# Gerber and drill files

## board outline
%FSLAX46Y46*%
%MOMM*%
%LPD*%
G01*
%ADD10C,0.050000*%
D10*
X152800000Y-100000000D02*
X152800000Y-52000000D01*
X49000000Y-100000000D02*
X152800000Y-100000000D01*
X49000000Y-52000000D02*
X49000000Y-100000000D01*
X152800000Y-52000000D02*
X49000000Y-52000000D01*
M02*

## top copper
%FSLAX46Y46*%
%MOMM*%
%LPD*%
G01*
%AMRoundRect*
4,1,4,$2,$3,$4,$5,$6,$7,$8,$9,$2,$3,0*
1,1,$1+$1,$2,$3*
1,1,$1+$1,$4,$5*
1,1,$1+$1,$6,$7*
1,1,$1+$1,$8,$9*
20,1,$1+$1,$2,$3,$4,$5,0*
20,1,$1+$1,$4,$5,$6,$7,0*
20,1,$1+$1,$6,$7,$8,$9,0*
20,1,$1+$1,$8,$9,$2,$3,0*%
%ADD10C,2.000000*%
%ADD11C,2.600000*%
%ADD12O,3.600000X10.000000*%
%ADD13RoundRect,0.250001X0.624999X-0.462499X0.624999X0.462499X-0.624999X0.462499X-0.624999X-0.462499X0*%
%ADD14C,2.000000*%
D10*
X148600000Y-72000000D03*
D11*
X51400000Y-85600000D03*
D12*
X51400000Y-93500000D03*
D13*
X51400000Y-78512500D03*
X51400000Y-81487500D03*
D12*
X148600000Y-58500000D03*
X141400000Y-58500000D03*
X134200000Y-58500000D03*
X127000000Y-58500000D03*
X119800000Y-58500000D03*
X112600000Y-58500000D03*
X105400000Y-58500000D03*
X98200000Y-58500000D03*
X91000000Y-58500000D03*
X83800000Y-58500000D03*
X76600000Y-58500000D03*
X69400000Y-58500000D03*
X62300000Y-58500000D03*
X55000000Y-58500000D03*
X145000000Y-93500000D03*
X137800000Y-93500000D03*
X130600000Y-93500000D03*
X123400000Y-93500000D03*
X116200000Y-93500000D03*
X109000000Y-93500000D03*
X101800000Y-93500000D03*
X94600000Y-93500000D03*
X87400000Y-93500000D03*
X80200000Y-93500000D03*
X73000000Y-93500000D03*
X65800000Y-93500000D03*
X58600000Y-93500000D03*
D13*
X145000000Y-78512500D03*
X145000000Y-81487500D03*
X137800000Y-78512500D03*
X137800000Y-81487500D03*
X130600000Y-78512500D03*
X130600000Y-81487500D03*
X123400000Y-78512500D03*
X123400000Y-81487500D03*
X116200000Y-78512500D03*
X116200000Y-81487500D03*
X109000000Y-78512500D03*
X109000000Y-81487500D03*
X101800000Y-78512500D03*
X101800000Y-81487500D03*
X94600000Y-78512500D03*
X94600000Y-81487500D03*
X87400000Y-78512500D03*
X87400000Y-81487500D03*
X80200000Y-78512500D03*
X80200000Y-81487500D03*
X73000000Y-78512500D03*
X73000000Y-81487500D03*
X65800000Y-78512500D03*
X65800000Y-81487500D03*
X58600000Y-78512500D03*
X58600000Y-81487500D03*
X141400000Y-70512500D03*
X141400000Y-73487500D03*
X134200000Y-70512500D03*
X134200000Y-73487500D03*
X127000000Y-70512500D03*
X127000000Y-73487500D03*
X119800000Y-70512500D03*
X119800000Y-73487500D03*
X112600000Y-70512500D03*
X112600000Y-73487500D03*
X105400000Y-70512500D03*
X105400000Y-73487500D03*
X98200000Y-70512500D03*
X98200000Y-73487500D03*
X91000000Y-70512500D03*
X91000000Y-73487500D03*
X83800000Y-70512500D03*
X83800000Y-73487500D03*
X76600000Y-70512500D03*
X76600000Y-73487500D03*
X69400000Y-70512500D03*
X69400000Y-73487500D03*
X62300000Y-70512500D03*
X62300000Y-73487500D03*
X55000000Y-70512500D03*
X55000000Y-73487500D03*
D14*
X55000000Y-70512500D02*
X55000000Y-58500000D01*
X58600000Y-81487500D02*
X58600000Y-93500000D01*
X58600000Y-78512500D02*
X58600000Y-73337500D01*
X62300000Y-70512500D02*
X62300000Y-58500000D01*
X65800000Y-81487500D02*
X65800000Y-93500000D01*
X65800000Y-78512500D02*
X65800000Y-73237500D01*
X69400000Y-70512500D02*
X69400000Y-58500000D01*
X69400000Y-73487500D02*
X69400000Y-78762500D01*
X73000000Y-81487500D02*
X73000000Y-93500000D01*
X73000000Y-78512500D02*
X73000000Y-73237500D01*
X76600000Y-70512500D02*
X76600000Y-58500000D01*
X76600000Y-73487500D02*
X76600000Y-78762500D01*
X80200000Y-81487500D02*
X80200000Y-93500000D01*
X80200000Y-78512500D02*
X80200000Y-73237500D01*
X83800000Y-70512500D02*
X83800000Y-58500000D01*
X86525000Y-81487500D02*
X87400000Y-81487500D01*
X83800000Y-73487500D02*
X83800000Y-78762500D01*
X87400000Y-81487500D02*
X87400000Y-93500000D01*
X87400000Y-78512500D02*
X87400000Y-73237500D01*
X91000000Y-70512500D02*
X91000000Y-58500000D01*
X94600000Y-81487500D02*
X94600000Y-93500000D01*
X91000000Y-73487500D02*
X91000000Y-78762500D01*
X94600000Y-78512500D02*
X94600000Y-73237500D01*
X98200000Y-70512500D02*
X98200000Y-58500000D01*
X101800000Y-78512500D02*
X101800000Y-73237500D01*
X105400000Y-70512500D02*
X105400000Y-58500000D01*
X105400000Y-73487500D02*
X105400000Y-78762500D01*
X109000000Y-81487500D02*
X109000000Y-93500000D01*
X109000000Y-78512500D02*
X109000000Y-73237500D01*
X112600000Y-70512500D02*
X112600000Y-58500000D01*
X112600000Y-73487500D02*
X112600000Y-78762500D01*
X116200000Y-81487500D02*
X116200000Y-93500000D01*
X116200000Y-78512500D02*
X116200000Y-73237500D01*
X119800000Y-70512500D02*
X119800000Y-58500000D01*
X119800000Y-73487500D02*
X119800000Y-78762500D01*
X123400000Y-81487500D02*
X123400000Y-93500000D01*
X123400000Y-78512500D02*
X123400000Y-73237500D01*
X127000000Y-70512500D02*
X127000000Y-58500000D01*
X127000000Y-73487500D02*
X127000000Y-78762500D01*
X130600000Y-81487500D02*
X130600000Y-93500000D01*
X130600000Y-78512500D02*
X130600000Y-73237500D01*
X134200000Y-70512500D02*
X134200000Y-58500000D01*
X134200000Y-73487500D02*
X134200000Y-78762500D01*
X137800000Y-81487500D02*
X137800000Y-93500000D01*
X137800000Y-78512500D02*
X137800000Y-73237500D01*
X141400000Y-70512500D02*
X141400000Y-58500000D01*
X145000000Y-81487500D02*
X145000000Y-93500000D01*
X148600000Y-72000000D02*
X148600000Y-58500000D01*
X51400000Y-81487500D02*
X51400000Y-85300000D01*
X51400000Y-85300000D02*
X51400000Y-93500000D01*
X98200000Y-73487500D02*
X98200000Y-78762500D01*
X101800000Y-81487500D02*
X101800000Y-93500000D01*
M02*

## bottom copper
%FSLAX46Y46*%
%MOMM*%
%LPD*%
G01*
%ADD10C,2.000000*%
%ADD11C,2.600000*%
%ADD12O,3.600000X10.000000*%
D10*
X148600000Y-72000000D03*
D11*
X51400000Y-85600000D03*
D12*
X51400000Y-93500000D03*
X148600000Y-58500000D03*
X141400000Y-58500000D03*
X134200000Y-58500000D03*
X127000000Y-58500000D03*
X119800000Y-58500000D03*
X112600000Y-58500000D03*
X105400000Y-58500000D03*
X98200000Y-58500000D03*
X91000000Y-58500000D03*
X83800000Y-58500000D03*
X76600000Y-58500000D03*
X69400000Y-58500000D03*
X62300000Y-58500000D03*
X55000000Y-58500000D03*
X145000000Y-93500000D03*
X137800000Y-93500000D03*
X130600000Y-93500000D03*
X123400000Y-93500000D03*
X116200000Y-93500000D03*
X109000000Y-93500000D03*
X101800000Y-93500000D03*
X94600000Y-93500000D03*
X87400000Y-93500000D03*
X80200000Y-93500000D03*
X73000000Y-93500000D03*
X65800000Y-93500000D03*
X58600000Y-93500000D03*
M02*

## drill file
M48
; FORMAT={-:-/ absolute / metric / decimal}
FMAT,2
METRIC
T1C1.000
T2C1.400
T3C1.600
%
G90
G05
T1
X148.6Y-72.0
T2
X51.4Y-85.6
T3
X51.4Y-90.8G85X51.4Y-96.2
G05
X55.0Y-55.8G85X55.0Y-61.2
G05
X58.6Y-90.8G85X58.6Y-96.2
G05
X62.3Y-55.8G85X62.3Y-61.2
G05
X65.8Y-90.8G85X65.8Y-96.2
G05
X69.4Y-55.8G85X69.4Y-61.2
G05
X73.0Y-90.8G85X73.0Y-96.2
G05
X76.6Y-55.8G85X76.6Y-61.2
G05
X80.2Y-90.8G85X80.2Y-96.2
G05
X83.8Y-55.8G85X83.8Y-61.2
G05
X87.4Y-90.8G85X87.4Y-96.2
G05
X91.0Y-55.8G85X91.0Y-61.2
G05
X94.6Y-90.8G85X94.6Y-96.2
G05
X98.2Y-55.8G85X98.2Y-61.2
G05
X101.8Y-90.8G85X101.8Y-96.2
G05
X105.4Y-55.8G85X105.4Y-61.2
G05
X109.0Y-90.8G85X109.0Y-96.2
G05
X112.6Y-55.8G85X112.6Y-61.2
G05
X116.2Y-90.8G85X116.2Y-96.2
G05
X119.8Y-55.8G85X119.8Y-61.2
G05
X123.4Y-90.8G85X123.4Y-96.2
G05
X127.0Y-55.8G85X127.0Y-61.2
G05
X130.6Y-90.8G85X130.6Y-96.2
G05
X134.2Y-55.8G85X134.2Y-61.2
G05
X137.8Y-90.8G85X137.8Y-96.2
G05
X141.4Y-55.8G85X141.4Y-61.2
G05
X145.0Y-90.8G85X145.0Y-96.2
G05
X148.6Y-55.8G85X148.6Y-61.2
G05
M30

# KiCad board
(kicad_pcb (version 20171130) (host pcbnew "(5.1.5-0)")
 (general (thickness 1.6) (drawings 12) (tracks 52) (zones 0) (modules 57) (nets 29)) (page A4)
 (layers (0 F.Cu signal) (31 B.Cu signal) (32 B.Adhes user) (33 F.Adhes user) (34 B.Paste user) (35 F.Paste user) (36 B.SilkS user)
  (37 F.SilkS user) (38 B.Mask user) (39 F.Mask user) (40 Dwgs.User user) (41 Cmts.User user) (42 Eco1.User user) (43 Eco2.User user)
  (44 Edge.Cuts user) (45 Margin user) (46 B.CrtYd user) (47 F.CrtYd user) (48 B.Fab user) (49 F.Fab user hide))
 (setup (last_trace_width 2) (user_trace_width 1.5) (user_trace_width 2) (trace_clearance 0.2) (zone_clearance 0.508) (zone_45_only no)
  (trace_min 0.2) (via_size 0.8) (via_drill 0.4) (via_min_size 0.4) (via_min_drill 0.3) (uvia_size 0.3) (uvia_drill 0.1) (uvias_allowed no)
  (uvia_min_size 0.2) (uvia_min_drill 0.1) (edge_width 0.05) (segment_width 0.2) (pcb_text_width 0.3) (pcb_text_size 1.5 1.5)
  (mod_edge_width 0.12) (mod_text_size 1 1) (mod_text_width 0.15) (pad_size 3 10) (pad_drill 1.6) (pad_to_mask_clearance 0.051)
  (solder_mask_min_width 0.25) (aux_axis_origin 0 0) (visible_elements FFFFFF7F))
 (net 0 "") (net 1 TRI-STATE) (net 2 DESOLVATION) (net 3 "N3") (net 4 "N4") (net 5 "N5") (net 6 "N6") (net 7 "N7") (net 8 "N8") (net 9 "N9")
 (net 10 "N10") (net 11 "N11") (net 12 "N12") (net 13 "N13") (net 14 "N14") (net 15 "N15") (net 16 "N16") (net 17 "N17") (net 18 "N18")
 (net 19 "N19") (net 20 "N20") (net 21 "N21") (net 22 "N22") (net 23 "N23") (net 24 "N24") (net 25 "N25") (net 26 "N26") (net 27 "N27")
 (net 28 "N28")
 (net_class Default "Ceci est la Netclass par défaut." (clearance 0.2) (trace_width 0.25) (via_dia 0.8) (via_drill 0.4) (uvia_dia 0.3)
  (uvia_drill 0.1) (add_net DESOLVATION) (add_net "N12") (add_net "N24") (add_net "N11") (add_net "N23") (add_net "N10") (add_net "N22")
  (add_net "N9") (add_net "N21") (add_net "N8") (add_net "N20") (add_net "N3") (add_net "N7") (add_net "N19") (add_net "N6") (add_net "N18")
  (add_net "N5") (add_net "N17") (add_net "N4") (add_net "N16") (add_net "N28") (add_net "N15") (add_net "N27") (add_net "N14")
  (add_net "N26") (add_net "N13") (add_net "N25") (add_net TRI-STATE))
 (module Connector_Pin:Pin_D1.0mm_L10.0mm (layer F.Cu) (at 148.6 72)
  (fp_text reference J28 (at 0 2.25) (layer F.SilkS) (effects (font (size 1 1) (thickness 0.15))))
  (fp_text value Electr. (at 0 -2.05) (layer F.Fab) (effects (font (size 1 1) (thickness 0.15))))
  (pad 1 thru_hole circle (at 0 0) (size 2 2) (drill 1) (layers *.Cu *.Mask) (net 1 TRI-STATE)))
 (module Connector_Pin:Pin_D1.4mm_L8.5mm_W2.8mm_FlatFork (layer F.Cu) (at 51.4 85.6 180)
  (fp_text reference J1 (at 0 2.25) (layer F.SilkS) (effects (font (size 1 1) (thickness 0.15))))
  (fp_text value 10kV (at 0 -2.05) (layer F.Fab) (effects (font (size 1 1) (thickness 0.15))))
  (pad 1 thru_hole circle (at 0 0 180) (size 2.6 2.6) (drill 1.4) (layers *.Cu *.Mask) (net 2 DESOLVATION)))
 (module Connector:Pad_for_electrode (layer F.Cu) (at 51.4 93.6)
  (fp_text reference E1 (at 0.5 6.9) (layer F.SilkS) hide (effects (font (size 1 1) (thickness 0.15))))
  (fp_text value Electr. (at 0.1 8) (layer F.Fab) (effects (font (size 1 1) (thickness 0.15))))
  (pad 1 thru_hole oval (at 0 -0.1) (size 3.6 10) (drill oval 1.6 7) (layers *.Cu *.Mask) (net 2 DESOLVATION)))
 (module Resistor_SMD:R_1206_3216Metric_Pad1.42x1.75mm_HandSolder (layer F.Cu) (at 51.4 80 90)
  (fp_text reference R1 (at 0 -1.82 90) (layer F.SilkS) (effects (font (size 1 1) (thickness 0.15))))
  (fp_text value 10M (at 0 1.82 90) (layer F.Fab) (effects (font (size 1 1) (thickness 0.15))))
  (pad 2 smd roundrect (at 1.4875 0 90) (size 1.425 1.75) (layers F.Cu F.Paste F.Mask) (roundrect_rratio 0.175439) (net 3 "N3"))
  (pad 1 smd roundrect (at -1.4875 0 90) (size 1.425 1.75) (layers F.Cu F.Paste F.Mask) (roundrect_rratio 0.175439) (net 2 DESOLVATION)))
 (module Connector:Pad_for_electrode (layer F.Cu) (at 148.6 58.6)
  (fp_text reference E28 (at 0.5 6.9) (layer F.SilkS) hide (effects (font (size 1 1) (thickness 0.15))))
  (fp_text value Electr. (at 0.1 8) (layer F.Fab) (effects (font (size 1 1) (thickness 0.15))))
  (pad 1 thru_hole oval (at 0 -0.1) (size 3.6 10) (drill oval 1.6 7) (layers *.Cu *.Mask) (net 1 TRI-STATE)))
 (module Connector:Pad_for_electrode (layer F.Cu) (at 141.4 58.6)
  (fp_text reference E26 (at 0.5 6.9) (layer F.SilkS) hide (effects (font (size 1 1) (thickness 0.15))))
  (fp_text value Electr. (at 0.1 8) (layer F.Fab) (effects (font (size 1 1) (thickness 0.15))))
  (pad 1 thru_hole oval (at 0 -0.1) (size 3.6 10) (drill oval 1.6 7) (layers *.Cu *.Mask) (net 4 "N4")))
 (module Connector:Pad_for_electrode (layer F.Cu) (at 134.2 58.6)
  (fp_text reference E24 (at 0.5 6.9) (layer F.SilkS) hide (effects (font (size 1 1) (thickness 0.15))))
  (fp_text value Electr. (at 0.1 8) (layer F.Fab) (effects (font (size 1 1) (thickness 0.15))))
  (pad 1 thru_hole oval (at 0 -0.1) (size 3.6 10) (drill oval 1.6 7) (layers *.Cu *.Mask) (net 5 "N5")))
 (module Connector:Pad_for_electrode (layer F.Cu) (at 127 58.6)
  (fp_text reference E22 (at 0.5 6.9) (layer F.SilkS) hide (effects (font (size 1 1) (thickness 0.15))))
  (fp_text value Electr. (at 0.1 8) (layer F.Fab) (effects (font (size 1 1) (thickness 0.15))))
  (pad 1 thru_hole oval (at 0 -0.1) (size 3.6 10) (drill oval 1.6 7) (layers *.Cu *.Mask) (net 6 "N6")))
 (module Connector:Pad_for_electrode (layer F.Cu) (at 119.8 58.6)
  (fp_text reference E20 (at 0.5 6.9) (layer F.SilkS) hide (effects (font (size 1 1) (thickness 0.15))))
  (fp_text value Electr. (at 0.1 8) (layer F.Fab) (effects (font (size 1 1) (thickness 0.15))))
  (pad 1 thru_hole oval (at 0 -0.1) (size 3.6 10) (drill oval 1.6 7) (layers *.Cu *.Mask) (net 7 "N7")))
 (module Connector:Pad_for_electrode (layer F.Cu) (at 112.6 58.6)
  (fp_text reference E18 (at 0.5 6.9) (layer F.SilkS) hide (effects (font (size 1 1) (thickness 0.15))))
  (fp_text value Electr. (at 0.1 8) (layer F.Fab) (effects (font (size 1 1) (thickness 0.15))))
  (pad 1 thru_hole oval (at 0 -0.1) (size 3.6 10) (drill oval 1.6 7) (layers *.Cu *.Mask) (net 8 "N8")))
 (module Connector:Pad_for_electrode (layer F.Cu) (at 105.4 58.6)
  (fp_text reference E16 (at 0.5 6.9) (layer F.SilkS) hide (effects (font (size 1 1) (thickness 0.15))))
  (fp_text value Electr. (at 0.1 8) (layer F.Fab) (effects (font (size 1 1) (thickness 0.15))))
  (pad 1 thru_hole oval (at 0 -0.1) (size 3.6 10) (drill oval 1.6 7) (layers *.Cu *.Mask) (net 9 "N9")))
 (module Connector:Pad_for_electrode (layer F.Cu) (at 98.2 58.6)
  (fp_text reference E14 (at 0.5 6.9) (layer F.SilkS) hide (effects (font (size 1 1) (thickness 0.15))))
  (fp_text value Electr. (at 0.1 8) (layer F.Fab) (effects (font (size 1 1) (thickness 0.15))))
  (pad 1 thru_hole oval (at 0 -0.1) (size 3.6 10) (drill oval 1.6 7) (layers *.Cu *.Mask) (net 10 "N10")))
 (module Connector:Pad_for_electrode (layer F.Cu) (at 91 58.6)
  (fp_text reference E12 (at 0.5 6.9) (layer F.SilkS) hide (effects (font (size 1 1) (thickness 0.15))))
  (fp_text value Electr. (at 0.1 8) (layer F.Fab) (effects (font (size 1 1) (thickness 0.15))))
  (pad 1 thru_hole oval (at 0 -0.1) (size 3.6 10) (drill oval 1.6 7) (layers *.Cu *.Mask) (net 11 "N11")))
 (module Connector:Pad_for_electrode (layer F.Cu) (at 83.8 58.6)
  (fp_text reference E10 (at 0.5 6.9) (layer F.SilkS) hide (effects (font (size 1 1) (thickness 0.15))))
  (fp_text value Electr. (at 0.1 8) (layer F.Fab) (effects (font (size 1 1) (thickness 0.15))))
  (pad 1 thru_hole oval (at 0 -0.1) (size 3.6 10) (drill oval 1.6 7) (layers *.Cu *.Mask) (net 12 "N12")))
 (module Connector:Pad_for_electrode (layer F.Cu) (at 76.6 58.6)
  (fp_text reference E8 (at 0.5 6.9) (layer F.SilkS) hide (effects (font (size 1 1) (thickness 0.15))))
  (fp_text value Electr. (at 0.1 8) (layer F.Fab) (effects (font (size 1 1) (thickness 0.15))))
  (pad 1 thru_hole oval (at 0 -0.1) (size 3.6 10) (drill oval 1.6 7) (layers *.Cu *.Mask) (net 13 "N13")))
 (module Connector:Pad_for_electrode (layer F.Cu) (at 69.4 58.6)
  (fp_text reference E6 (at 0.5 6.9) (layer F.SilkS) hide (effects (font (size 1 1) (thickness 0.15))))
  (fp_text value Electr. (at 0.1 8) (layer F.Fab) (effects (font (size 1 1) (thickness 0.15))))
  (pad 1 thru_hole oval (at 0 -0.1) (size 3.6 10) (drill oval 1.6 7) (layers *.Cu *.Mask) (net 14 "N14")))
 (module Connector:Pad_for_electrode (layer F.Cu) (at 62.3 58.6)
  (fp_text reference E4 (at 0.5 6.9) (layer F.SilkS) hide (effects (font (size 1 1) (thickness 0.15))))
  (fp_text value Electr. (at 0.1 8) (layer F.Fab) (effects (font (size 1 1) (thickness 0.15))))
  (pad 1 thru_hole oval (at 0 -0.1) (size 3.6 10) (drill oval 1.6 7) (layers *.Cu *.Mask) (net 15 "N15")))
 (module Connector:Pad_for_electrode (layer F.Cu) (at 55 58.6)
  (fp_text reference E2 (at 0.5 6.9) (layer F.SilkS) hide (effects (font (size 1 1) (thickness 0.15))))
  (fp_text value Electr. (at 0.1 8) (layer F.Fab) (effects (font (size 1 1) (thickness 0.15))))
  (pad 1 thru_hole oval (at 0 -0.1) (size 3.6 10) (drill oval 1.6 7) (layers *.Cu *.Mask) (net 3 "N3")))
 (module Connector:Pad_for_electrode (layer F.Cu) (at 145 93.6)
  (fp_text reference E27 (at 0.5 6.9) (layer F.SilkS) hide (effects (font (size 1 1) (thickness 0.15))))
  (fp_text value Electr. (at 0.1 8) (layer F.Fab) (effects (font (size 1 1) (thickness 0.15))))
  (pad 1 thru_hole oval (at 0 -0.1) (size 3.6 10) (drill oval 1.6 7) (layers *.Cu *.Mask) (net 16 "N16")))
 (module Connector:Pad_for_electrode (layer F.Cu) (at 137.8 93.6)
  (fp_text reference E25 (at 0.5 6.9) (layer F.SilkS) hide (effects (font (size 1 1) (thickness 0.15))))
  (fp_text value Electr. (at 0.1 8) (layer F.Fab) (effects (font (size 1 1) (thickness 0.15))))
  (pad 1 thru_hole oval (at 0 -0.1) (size 3.6 10) (drill oval 1.6 7) (layers *.Cu *.Mask) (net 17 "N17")))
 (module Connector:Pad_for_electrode (layer F.Cu) (at 130.6 93.6)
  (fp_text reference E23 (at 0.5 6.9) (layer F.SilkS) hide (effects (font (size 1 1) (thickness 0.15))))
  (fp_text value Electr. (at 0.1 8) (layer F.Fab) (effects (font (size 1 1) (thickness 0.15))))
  (pad 1 thru_hole oval (at 0 -0.1) (size 3.6 10) (drill oval 1.6 7) (layers *.Cu *.Mask) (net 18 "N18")))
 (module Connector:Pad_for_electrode (layer F.Cu) (at 123.4 93.6)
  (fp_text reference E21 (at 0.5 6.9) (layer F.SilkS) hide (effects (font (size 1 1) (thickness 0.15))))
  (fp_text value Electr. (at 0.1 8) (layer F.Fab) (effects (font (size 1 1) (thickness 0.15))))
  (pad 1 thru_hole oval (at 0 -0.1) (size 3.6 10) (drill oval 1.6 7) (layers *.Cu *.Mask) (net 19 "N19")))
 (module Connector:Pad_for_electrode (layer F.Cu) (at 116.2 93.6)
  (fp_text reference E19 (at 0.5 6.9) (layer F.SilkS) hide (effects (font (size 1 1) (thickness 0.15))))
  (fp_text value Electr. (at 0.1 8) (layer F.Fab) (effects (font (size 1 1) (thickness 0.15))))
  (pad 1 thru_hole oval (at 0 -0.1) (size 3.6 10) (drill oval 1.6 7) (layers *.Cu *.Mask) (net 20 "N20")))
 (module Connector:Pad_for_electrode (layer F.Cu) (at 109 93.6)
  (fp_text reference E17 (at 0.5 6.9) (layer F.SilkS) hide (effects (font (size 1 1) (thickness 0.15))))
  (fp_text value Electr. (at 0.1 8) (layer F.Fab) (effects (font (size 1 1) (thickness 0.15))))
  (pad 1 thru_hole oval (at 0 -0.1) (size 3.6 10) (drill oval 1.6 7) (layers *.Cu *.Mask) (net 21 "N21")))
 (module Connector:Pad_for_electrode (layer F.Cu) (at 101.8 93.6)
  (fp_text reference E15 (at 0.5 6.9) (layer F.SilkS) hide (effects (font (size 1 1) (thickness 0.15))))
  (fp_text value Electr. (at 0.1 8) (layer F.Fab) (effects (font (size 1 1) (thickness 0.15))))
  (pad 1 thru_hole oval (at 0 -0.1) (size 3.6 10) (drill oval 1.6 7) (layers *.Cu *.Mask) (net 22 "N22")))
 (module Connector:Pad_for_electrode (layer F.Cu) (at 94.6 93.6)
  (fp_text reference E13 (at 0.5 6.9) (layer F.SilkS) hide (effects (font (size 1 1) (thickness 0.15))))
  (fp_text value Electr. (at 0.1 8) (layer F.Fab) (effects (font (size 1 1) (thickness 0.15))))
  (pad 1 thru_hole oval (at 0 -0.1) (size 3.6 10) (drill oval 1.6 7) (layers *.Cu *.Mask) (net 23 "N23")))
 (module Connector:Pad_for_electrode (layer F.Cu) (at 87.4 93.6)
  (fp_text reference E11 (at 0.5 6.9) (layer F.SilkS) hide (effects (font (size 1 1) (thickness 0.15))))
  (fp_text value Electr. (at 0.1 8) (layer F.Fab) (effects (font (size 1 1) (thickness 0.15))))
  (pad 1 thru_hole oval (at 0 -0.1) (size 3.6 10) (drill oval 1.6 7) (layers *.Cu *.Mask) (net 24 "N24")))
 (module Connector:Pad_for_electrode (layer F.Cu) (at 80.2 93.6)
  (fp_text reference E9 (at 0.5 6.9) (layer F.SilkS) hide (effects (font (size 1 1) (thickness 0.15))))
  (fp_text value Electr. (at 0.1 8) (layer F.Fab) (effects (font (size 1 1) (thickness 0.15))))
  (pad 1 thru_hole oval (at 0 -0.1) (size 3.6 10) (drill oval 1.6 7) (layers *.Cu *.Mask) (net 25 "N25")))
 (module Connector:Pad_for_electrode (layer F.Cu) (at 73 93.6)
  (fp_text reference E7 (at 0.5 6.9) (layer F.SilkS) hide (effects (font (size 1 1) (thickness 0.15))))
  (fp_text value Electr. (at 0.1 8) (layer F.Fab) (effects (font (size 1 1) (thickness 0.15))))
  (pad 1 thru_hole oval (at 0 -0.1) (size 3.6 10) (drill oval 1.6 7) (layers *.Cu *.Mask) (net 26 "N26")))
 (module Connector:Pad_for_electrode (layer F.Cu) (at 65.8 93.6)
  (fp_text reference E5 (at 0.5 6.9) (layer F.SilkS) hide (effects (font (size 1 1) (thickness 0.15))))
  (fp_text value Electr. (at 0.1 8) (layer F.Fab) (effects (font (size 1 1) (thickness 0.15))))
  (pad 1 thru_hole oval (at 0 -0.1) (size 3.6 10) (drill oval 1.6 7) (layers *.Cu *.Mask) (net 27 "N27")))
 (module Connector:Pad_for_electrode (layer F.Cu) (at 58.6 93.6)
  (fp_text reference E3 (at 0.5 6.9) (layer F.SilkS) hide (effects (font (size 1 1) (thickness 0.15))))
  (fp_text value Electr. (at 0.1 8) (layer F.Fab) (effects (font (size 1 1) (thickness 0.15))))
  (pad 1 thru_hole oval (at 0 -0.1) (size 3.6 10) (drill oval 1.6 7) (layers *.Cu *.Mask) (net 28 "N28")))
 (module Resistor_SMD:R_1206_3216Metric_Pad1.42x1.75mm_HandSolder (layer F.Cu) (at 145 80 90)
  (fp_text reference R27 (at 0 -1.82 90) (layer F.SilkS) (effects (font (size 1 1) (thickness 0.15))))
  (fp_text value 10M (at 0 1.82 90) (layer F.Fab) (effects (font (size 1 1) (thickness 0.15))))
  (pad 2 smd roundrect (at 1.4875 0 90) (size 1.425 1.75) (layers F.Cu F.Paste F.Mask) (roundrect_rratio 0.175439) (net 1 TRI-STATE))
  (pad 1 smd roundrect (at -1.4875 0 90) (size 1.425 1.75) (layers F.Cu F.Paste F.Mask) (roundrect_rratio 0.175439) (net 16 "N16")))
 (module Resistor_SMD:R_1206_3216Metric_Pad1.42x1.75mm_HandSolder (layer F.Cu) (at 137.8 80 90)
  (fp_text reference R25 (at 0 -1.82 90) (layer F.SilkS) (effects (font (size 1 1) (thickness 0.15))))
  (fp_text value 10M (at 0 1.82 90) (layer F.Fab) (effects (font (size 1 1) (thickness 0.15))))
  (pad 2 smd roundrect (at 1.4875 0 90) (size 1.425 1.75) (layers F.Cu F.Paste F.Mask) (roundrect_rratio 0.175439) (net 4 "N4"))
  (pad 1 smd roundrect (at -1.4875 0 90) (size 1.425 1.75) (layers F.Cu F.Paste F.Mask) (roundrect_rratio 0.175439) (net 17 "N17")))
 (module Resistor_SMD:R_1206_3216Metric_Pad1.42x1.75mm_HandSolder (layer F.Cu) (at 130.6 80 90)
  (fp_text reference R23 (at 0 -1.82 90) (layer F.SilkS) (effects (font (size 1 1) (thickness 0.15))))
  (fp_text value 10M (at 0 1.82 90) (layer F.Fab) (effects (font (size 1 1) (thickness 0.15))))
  (pad 2 smd roundrect (at 1.4875 0 90) (size 1.425 1.75) (layers F.Cu F.Paste F.Mask) (roundrect_rratio 0.175439) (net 5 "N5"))
  (pad 1 smd roundrect (at -1.4875 0 90) (size 1.425 1.75) (layers F.Cu F.Paste F.Mask) (roundrect_rratio 0.175439) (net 18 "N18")))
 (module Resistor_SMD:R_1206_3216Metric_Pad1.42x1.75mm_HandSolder (layer F.Cu) (at 123.4 80 90)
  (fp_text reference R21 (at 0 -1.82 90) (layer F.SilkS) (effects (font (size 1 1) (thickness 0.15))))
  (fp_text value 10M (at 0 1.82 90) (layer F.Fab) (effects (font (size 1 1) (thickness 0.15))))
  (pad 2 smd roundrect (at 1.4875 0 90) (size 1.425 1.75) (layers F.Cu F.Paste F.Mask) (roundrect_rratio 0.175439) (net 6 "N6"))
  (pad 1 smd roundrect (at -1.4875 0 90) (size 1.425 1.75) (layers F.Cu F.Paste F.Mask) (roundrect_rratio 0.175439) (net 19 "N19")))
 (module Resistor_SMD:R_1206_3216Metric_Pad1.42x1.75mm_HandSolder (layer F.Cu) (at 116.2 80 90)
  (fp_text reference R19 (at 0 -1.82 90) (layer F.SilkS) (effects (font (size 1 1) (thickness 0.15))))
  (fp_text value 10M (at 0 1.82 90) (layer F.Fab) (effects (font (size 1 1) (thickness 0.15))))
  (pad 2 smd roundrect (at 1.4875 0 90) (size 1.425 1.75) (layers F.Cu F.Paste F.Mask) (roundrect_rratio 0.175439) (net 7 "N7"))
  (pad 1 smd roundrect (at -1.4875 0 90) (size 1.425 1.75) (layers F.Cu F.Paste F.Mask) (roundrect_rratio 0.175439) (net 20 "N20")))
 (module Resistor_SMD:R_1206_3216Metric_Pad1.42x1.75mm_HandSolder (layer F.Cu) (at 109 80 90)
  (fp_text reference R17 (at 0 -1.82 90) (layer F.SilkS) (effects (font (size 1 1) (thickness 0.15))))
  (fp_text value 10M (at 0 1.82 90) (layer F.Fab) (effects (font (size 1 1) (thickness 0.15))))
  (pad 2 smd roundrect (at 1.4875 0 90) (size 1.425 1.75) (layers F.Cu F.Paste F.Mask) (roundrect_rratio 0.175439) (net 8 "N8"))
  (pad 1 smd roundrect (at -1.4875 0 90) (size 1.425 1.75) (layers F.Cu F.Paste F.Mask) (roundrect_rratio 0.175439) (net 21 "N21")))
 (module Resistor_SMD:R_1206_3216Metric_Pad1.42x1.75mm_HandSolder (layer F.Cu) (at 101.8 80 90)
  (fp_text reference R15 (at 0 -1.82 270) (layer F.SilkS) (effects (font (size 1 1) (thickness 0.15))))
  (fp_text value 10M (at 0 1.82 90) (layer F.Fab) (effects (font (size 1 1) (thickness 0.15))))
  (pad 2 smd roundrect (at 1.4875 0 90) (size 1.425 1.75) (layers F.Cu F.Paste F.Mask) (roundrect_rratio 0.175439) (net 9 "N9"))
  (pad 1 smd roundrect (at -1.4875 0 90) (size 1.425 1.75) (layers F.Cu F.Paste F.Mask) (roundrect_rratio 0.175439) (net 22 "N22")))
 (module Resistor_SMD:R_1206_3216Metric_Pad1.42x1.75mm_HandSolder (layer F.Cu) (at 94.6 80 90)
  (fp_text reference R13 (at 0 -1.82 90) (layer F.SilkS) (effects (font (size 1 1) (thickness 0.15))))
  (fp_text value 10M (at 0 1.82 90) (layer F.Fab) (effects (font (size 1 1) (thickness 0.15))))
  (pad 2 smd roundrect (at 1.4875 0 90) (size 1.425 1.75) (layers F.Cu F.Paste F.Mask) (roundrect_rratio 0.175439) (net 10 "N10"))
  (pad 1 smd roundrect (at -1.4875 0 90) (size 1.425 1.75) (layers F.Cu F.Paste F.Mask) (roundrect_rratio 0.175439) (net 23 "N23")))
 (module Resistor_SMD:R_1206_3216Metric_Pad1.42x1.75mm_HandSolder (layer F.Cu) (at 87.4 80 90)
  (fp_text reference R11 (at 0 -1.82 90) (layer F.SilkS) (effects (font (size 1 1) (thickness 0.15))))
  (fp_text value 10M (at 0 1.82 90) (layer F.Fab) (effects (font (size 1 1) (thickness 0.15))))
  (pad 2 smd roundrect (at 1.4875 0 90) (size 1.425 1.75) (layers F.Cu F.Paste F.Mask) (roundrect_rratio 0.175439) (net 11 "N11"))
  (pad 1 smd roundrect (at -1.4875 0 90) (size 1.425 1.75) (layers F.Cu F.Paste F.Mask) (roundrect_rratio 0.175439) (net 24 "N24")))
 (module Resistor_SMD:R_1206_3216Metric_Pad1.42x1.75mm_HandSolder (layer F.Cu) (at 80.2 80 90)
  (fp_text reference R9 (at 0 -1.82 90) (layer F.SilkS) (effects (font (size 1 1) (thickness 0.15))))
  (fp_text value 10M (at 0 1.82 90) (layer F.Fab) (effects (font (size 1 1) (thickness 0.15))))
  (pad 2 smd roundrect (at 1.4875 0 90) (size 1.425 1.75) (layers F.Cu F.Paste F.Mask) (roundrect_rratio 0.175439) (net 12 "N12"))
  (pad 1 smd roundrect (at -1.4875 0 90) (size 1.425 1.75) (layers F.Cu F.Paste F.Mask) (roundrect_rratio 0.175439) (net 25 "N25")))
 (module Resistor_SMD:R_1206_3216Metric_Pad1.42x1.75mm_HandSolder (layer F.Cu) (at 73 80 90)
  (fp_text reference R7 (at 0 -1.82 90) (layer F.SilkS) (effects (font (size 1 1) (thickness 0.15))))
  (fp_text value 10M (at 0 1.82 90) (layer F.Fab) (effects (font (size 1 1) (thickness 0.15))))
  (pad 2 smd roundrect (at 1.4875 0 90) (size 1.425 1.75) (layers F.Cu F.Paste F.Mask) (roundrect_rratio 0.175439) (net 13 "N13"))
  (pad 1 smd roundrect (at -1.4875 0 90) (size 1.425 1.75) (layers F.Cu F.Paste F.Mask) (roundrect_rratio 0.175439) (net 26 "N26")))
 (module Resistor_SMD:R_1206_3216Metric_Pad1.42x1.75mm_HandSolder (layer F.Cu) (at 65.8 80 90)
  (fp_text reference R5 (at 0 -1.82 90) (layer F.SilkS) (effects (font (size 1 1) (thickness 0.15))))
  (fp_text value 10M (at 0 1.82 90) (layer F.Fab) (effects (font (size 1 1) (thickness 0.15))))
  (pad 2 smd roundrect (at 1.4875 0 90) (size 1.425 1.75) (layers F.Cu F.Paste F.Mask) (roundrect_rratio 0.175439) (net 14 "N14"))
  (pad 1 smd roundrect (at -1.4875 0 90) (size 1.425 1.75) (layers F.Cu F.Paste F.Mask) (roundrect_rratio 0.175439) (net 27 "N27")))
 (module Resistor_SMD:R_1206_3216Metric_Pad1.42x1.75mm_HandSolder (layer F.Cu) (at 58.6 80 90)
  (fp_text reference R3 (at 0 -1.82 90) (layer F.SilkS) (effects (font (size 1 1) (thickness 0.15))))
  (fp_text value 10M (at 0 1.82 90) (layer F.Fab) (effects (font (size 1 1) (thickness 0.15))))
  (pad 2 smd roundrect (at 1.4875 0 90) (size 1.425 1.75) (layers F.Cu F.Paste F.Mask) (roundrect_rratio 0.175439) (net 15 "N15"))
  (pad 1 smd roundrect (at -1.4875 0 90) (size 1.425 1.75) (layers F.Cu F.Paste F.Mask) (roundrect_rratio 0.175439) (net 28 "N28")))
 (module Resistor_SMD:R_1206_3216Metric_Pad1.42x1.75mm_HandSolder (layer F.Cu) (at 141.4 72 90)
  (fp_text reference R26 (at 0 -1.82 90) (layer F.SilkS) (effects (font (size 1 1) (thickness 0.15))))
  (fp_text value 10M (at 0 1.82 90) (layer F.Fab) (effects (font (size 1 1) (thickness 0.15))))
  (pad 2 smd roundrect (at 1.4875 0 90) (size 1.425 1.75) (layers F.Cu F.Paste F.Mask) (roundrect_rratio 0.175439) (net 4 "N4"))
  (pad 1 smd roundrect (at -1.4875 0 90) (size 1.425 1.75) (layers F.Cu F.Paste F.Mask) (roundrect_rratio 0.175439) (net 16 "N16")))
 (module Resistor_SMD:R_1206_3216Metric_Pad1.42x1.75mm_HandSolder (layer F.Cu) (at 134.2 72 90)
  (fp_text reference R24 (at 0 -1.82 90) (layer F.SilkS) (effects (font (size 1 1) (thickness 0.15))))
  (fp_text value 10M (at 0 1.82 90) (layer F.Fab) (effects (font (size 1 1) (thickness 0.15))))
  (pad 2 smd roundrect (at 1.4875 0 90) (size 1.425 1.75) (layers F.Cu F.Paste F.Mask) (roundrect_rratio 0.175439) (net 5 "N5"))
  (pad 1 smd roundrect (at -1.4875 0 90) (size 1.425 1.75) (layers F.Cu F.Paste F.Mask) (roundrect_rratio 0.175439) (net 17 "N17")))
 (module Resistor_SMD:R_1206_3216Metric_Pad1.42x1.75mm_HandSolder (layer F.Cu) (at 127 72 90)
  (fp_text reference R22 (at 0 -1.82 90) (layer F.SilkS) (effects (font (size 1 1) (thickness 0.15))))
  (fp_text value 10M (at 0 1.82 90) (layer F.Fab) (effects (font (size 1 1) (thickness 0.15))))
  (pad 2 smd roundrect (at 1.4875 0 90) (size 1.425 1.75) (layers F.Cu F.Paste F.Mask) (roundrect_rratio 0.175439) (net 6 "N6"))
  (pad 1 smd roundrect (at -1.4875 0 90) (size 1.425 1.75) (layers F.Cu F.Paste F.Mask) (roundrect_rratio 0.175439) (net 18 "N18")))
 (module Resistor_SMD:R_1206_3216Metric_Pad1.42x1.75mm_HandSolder (layer F.Cu) (at 119.8 72 90)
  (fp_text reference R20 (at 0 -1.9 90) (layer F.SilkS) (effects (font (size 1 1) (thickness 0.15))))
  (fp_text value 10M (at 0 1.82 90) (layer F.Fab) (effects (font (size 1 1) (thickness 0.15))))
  (pad 2 smd roundrect (at 1.4875 0 90) (size 1.425 1.75) (layers F.Cu F.Paste F.Mask) (roundrect_rratio 0.175439) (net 7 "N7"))
  (pad 1 smd roundrect (at -1.4875 0 90) (size 1.425 1.75) (layers F.Cu F.Paste F.Mask) (roundrect_rratio 0.175439) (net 19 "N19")))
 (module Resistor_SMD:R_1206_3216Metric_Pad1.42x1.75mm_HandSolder (layer F.Cu) (at 112.6 72 90)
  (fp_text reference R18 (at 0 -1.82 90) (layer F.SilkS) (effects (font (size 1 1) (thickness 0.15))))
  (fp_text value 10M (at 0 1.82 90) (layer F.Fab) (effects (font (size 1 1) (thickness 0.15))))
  (pad 2 smd roundrect (at 1.4875 0 90) (size 1.425 1.75) (layers F.Cu F.Paste F.Mask) (roundrect_rratio 0.175439) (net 8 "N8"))
  (pad 1 smd roundrect (at -1.4875 0 90) (size 1.425 1.75) (layers F.Cu F.Paste F.Mask) (roundrect_rratio 0.175439) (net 20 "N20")))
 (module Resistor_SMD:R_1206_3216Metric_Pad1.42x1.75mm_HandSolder (layer F.Cu) (at 105.4 72 90)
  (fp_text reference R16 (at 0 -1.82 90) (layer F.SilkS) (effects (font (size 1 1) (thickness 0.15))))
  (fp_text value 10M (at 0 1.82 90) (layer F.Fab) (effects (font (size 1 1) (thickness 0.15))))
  (pad 2 smd roundrect (at 1.4875 0 90) (size 1.425 1.75) (layers F.Cu F.Paste F.Mask) (roundrect_rratio 0.175439) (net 9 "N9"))
  (pad 1 smd roundrect (at -1.4875 0 90) (size 1.425 1.75) (layers F.Cu F.Paste F.Mask) (roundrect_rratio 0.175439) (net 21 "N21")))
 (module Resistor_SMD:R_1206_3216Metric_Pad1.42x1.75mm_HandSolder (layer F.Cu) (at 98.2 72 90)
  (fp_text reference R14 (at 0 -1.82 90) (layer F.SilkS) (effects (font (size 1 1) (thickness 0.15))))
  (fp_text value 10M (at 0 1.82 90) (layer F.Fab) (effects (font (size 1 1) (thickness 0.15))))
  (pad 2 smd roundrect (at 1.4875 0 90) (size 1.425 1.75) (layers F.Cu F.Paste F.Mask) (roundrect_rratio 0.175439) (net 10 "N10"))
  (pad 1 smd roundrect (at -1.4875 0 90) (size 1.425 1.75) (layers F.Cu F.Paste F.Mask) (roundrect_rratio 0.175439) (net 22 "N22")))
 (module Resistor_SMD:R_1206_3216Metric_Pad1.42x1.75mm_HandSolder (layer F.Cu) (at 91 72 90)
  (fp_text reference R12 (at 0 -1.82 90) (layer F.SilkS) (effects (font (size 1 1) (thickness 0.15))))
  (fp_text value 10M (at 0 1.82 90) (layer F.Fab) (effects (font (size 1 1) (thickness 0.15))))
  (pad 2 smd roundrect (at 1.4875 0 90) (size 1.425 1.75) (layers F.Cu F.Paste F.Mask) (roundrect_rratio 0.175439) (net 11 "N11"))
  (pad 1 smd roundrect (at -1.4875 0 90) (size 1.425 1.75) (layers F.Cu F.Paste F.Mask) (roundrect_rratio 0.175439) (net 23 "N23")))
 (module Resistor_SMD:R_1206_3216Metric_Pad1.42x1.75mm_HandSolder (layer F.Cu) (at 83.8 72 90)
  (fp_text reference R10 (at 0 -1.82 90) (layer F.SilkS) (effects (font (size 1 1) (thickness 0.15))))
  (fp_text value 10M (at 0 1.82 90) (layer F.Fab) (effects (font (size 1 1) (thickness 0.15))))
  (pad 2 smd roundrect (at 1.4875 0 90) (size 1.425 1.75) (layers F.Cu F.Paste F.Mask) (roundrect_rratio 0.175439) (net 12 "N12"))
  (pad 1 smd roundrect (at -1.4875 0 90) (size 1.425 1.75) (layers F.Cu F.Paste F.Mask) (roundrect_rratio 0.175439) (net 24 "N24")))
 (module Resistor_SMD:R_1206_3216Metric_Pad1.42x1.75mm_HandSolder (layer F.Cu) (at 76.6 72 90)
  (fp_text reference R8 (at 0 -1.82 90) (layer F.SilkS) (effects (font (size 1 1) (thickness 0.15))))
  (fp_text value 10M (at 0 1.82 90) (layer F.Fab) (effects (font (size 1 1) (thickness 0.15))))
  (pad 2 smd roundrect (at 1.4875 0 90) (size 1.425 1.75) (layers F.Cu F.Paste F.Mask) (roundrect_rratio 0.175439) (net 13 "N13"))
  (pad 1 smd roundrect (at -1.4875 0 90) (size 1.425 1.75) (layers F.Cu F.Paste F.Mask) (roundrect_rratio 0.175439) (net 25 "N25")))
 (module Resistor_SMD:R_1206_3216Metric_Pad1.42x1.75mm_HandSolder (layer F.Cu) (at 69.4 72 90)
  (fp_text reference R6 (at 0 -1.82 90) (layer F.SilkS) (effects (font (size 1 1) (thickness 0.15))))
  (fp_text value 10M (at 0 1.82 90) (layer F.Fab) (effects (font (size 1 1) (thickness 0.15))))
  (pad 2 smd roundrect (at 1.4875 0 90) (size 1.425 1.75) (layers F.Cu F.Paste F.Mask) (roundrect_rratio 0.175439) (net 14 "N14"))
  (pad 1 smd roundrect (at -1.4875 0 90) (size 1.425 1.75) (layers F.Cu F.Paste F.Mask) (roundrect_rratio 0.175439) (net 26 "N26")))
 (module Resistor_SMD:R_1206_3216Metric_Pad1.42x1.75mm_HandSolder (layer F.Cu) (at 62.3 72 90)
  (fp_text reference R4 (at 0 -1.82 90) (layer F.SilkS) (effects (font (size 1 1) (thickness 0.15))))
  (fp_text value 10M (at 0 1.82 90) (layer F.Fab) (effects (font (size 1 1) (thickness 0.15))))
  (pad 2 smd roundrect (at 1.4875 0 90) (size 1.425 1.75) (layers F.Cu F.Paste F.Mask) (roundrect_rratio 0.175439) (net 15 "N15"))
  (pad 1 smd roundrect (at -1.4875 0 90) (size 1.425 1.75) (layers F.Cu F.Paste F.Mask) (roundrect_rratio 0.175439) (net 27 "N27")))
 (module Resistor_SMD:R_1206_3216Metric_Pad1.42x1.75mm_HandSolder (layer F.Cu) (at 55 72 90)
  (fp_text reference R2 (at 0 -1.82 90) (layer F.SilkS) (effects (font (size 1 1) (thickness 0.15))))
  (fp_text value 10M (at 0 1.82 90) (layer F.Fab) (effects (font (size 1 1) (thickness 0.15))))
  (pad 2 smd roundrect (at 1.4875 0 90) (size 1.425 1.75) (layers F.Cu F.Paste F.Mask) (roundrect_rratio 0.175439) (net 3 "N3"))
  (pad 1 smd roundrect (at -1.4875 0 90) (size 1.425 1.75) (layers F.Cu F.Paste F.Mask) (roundrect_rratio 0.175439) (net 28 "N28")))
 (gr_line (start 152.8 100) (end 152.8 52) (layer Edge.Cuts) (width 0.05))
 (gr_line (start 49 100) (end 152.8 100) (layer Edge.Cuts) (width 0.05))
 (gr_line (start 49 52) (end 49 100) (layer Edge.Cuts) (width 0.05))
 (gr_line (start 152.8 52) (end 49 52) (layer Edge.Cuts) (width 0.05))
 (segment (start 55 70.5125) (end 55 58.5) (width 2) (layer F.Cu) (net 3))
 (segment (start 58.6 81.4875) (end 58.6 93.5) (width 2) (layer F.Cu) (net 28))
 (segment (start 58.6 78.5125) (end 58.6 73.3375) (width 2) (layer F.Cu) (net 15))
 (segment (start 62.3 70.5125) (end 62.3 58.5) (width 2) (layer F.Cu) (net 15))
 (segment (start 65.8 81.4875) (end 65.8 93.5) (width 2) (layer F.Cu) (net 27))
 (segment (start 65.8 78.5125) (end 65.8 73.2375) (width 2) (layer F.Cu) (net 14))
 (segment (start 69.4 70.5125) (end 69.4 58.5) (width 2) (layer F.Cu) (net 14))
 (segment (start 69.4 73.4875) (end 69.4 78.7625) (width 2) (layer F.Cu) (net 26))
 (segment (start 73 81.4875) (end 73 93.5) (width 2) (layer F.Cu) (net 26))
 (segment (start 73 78.5125) (end 73 73.2375) (width 2) (layer F.Cu) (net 13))
 (segment (start 76.6 70.5125) (end 76.6 58.5) (width 2) (layer F.Cu) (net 13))
 (segment (start 76.6 73.4875) (end 76.6 78.7625) (width 2) (layer F.Cu) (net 25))
 (segment (start 80.2 81.4875) (end 80.2 93.5) (width 2) (layer F.Cu) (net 25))
 (segment (start 80.2 78.5125) (end 80.2 73.2375) (width 2) (layer F.Cu) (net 12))
 (segment (start 83.8 70.5125) (end 83.8 58.5) (width 2) (layer F.Cu) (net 12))
 (segment (start 86.525 81.4875) (end 87.4 81.4875) (width 2) (layer F.Cu) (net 24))
 (segment (start 83.8 73.4875) (end 83.8 78.7625) (width 2) (layer F.Cu) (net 24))
 (segment (start 87.4 81.4875) (end 87.4 93.5) (width 2) (layer F.Cu) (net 24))
 (segment (start 87.4 78.5125) (end 87.4 73.2375) (width 2) (layer F.Cu) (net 11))
 (segment (start 91 70.5125) (end 91 58.5) (width 2) (layer F.Cu) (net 11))
 (segment (start 94.6 81.4875) (end 94.6 93.5) (width 2) (layer F.Cu) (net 23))
 (segment (start 91 73.4875) (end 91 78.7625) (width 2) (layer F.Cu) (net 23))
 (segment (start 94.6 78.5125) (end 94.6 73.2375) (width 2) (layer F.Cu) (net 10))
 (segment (start 98.2 70.5125) (end 98.2 58.5) (width 2) (layer F.Cu) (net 10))
 (segment (start 101.8 78.5125) (end 101.8 73.2375) (width 2) (layer F.Cu) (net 9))
 (segment (start 105.4 70.5125) (end 105.4 58.5) (width 2) (layer F.Cu) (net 9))
 (segment (start 105.4 73.4875) (end 105.4 78.7625) (width 2) (layer F.Cu) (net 21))
 (segment (start 109 81.4875) (end 109 93.5) (width 2) (layer F.Cu) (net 21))
 (segment (start 109 78.5125) (end 109 73.2375) (width 2) (layer F.Cu) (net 8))
 (segment (start 112.6 70.5125) (end 112.6 58.5) (width 2) (layer F.Cu) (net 8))
 (segment (start 112.6 73.4875) (end 112.6 78.7625) (width 2) (layer F.Cu) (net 20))
 (segment (start 116.2 81.4875) (end 116.2 93.5) (width 2) (layer F.Cu) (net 20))
 (segment (start 116.2 78.5125) (end 116.2 73.2375) (width 2) (layer F.Cu) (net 7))
 (segment (start 119.8 70.5125) (end 119.8 58.5) (width 2) (layer F.Cu) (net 7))
 (segment (start 119.8 73.4875) (end 119.8 78.7625) (width 2) (layer F.Cu) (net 19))
 (segment (start 123.4 81.4875) (end 123.4 93.5) (width 2) (layer F.Cu) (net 19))
 (segment (start 123.4 78.5125) (end 123.4 73.2375) (width 2) (layer F.Cu) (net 6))
 (segment (start 127 70.5125) (end 127 58.5) (width 2) (layer F.Cu) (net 6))
 (segment (start 127 73.4875) (end 127 78.7625) (width 2) (layer F.Cu) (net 18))
 (segment (start 130.6 81.4875) (end 130.6 93.5) (width 2) (layer F.Cu) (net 18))
 (segment (start 130.6 78.5125) (end 130.6 73.2375) (width 2) (layer F.Cu) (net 5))
 (segment (start 134.2 70.5125) (end 134.2 58.5) (width 2) (layer F.Cu) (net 5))
 (segment (start 134.2 73.4875) (end 134.2 78.7625) (width 2) (layer F.Cu) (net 17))
 (segment (start 137.8 81.4875) (end 137.8 93.5) (width 2) (layer F.Cu) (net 17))
 (segment (start 137.8 78.5125) (end 137.8 73.2375) (width 2) (layer F.Cu) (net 4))
 (segment (start 141.4 70.5125) (end 141.4 58.5) (width 2) (layer F.Cu) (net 4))
 (segment (start 145 81.4875) (end 145 93.5) (width 2) (layer F.Cu) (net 16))
 (segment (start 148.6 72) (end 148.6 58.5) (width 2) (layer F.Cu) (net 1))
 (segment (start 51.4 81.4875) (end 51.4 85.3) (width 2) (layer F.Cu) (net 2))
 (segment (start 51.4 85.3) (end 51.4 93.5) (width 2) (layer F.Cu) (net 2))
 (segment (start 98.2 73.4875) (end 98.2 78.7625) (width 2) (layer F.Cu) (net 22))
 (segment (start 101.8 81.4875) (end 101.8 93.5) (width 2) (layer F.Cu) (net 22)))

